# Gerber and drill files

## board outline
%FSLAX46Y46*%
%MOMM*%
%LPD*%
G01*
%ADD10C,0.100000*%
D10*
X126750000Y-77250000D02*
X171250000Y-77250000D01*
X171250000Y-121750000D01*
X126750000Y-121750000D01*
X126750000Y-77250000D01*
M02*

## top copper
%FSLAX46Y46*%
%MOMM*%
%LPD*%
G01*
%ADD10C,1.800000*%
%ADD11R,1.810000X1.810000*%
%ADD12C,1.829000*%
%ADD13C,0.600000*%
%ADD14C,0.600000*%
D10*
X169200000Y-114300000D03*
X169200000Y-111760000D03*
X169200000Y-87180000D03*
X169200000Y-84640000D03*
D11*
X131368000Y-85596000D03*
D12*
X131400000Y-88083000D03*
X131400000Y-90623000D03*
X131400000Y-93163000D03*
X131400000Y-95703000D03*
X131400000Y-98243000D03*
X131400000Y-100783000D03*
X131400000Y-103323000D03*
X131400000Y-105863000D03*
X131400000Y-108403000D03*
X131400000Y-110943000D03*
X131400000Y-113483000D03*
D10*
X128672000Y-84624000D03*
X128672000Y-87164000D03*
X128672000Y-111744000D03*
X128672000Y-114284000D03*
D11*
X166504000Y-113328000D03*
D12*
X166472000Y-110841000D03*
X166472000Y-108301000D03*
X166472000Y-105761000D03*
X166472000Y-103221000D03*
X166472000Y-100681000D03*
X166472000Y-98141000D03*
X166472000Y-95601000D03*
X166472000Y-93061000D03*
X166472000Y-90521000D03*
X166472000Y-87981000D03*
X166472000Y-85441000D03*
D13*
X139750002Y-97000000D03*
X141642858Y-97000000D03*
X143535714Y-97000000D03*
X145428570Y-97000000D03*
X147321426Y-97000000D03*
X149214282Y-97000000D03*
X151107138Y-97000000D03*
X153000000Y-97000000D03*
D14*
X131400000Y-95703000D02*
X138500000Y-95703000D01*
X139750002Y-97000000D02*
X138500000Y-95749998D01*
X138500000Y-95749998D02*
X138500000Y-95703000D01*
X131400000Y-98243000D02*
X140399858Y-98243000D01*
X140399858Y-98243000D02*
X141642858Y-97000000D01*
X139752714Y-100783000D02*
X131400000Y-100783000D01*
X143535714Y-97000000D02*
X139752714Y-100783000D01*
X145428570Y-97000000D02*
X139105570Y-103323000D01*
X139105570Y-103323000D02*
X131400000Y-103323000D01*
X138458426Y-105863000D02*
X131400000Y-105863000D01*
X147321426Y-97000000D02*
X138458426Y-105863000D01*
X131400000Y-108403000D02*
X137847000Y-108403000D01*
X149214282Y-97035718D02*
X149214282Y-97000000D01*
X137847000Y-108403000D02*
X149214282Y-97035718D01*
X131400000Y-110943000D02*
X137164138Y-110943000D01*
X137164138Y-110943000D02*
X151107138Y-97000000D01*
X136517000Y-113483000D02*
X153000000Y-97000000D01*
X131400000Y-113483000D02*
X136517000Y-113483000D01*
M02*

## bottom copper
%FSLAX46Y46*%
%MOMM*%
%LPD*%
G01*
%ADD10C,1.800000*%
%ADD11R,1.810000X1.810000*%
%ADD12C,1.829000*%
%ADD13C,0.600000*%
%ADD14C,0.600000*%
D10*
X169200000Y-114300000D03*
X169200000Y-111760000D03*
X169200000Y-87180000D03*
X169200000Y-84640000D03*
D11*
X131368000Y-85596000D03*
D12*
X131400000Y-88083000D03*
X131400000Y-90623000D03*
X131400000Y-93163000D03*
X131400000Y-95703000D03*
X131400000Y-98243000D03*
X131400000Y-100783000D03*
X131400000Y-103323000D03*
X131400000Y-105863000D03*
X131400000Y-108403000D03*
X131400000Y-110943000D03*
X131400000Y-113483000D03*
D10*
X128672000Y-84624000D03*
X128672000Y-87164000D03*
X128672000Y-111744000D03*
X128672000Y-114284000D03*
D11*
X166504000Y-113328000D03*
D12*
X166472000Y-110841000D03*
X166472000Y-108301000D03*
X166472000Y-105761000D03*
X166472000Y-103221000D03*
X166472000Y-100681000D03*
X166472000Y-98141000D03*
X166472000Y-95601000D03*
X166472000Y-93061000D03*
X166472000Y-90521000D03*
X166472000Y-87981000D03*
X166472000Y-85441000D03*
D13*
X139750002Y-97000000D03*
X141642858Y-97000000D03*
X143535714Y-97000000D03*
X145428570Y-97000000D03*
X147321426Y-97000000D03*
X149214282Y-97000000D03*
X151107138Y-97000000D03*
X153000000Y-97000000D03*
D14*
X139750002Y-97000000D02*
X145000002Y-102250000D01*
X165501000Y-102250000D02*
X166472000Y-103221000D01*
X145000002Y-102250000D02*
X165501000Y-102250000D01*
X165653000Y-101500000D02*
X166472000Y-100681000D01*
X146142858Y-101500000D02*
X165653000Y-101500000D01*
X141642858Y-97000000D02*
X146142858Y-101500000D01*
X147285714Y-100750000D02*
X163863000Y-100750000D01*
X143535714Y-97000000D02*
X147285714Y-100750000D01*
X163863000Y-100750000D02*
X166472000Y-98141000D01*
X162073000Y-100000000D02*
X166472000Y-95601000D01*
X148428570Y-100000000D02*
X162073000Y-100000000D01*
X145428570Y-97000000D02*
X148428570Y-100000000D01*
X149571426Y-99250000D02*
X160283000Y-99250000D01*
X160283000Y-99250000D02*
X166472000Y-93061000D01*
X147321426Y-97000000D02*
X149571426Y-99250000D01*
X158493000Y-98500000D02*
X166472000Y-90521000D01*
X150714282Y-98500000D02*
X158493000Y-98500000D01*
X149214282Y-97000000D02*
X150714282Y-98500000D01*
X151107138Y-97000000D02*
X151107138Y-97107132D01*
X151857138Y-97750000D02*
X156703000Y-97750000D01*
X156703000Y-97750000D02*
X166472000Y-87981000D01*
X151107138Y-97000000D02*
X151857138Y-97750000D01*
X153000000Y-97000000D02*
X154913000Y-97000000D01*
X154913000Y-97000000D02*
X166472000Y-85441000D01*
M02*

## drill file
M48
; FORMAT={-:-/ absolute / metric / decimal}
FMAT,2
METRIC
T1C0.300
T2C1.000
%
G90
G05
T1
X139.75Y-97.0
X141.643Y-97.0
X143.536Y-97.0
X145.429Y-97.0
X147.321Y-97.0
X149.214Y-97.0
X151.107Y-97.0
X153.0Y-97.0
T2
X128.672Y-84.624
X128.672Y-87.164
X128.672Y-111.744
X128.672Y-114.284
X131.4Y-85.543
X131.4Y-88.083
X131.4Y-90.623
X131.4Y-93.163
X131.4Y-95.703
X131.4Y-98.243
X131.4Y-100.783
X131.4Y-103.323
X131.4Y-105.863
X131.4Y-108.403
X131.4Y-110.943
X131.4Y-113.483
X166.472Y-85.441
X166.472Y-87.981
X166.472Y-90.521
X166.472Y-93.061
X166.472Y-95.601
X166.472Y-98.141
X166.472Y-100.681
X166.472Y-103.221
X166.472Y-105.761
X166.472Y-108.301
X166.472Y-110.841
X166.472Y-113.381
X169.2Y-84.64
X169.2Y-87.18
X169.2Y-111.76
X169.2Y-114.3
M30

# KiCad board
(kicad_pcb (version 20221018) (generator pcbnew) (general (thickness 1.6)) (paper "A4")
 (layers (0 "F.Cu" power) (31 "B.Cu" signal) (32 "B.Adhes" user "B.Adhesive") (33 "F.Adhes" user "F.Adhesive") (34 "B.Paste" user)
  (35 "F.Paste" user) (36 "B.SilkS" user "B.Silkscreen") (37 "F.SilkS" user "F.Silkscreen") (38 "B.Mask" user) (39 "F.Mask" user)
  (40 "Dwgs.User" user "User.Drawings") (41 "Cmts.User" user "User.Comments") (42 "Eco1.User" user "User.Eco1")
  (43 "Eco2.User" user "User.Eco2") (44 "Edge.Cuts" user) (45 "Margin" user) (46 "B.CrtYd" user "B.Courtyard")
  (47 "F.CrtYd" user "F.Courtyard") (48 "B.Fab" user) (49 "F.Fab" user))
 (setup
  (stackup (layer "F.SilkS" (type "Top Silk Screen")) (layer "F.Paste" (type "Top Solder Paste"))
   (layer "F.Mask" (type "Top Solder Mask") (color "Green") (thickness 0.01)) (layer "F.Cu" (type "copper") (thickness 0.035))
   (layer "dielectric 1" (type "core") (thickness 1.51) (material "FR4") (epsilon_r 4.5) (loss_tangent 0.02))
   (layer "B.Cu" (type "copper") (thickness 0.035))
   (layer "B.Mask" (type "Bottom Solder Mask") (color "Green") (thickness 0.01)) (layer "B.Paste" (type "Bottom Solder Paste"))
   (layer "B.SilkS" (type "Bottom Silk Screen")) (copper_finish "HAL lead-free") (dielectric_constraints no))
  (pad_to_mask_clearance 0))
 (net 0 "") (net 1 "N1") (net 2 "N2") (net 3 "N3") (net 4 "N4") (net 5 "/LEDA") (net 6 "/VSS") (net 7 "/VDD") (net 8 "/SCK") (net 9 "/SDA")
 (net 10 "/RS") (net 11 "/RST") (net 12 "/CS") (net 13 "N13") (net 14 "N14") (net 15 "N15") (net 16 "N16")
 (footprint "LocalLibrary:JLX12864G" (layer "F.Cu") (at 148.936 99.462 90)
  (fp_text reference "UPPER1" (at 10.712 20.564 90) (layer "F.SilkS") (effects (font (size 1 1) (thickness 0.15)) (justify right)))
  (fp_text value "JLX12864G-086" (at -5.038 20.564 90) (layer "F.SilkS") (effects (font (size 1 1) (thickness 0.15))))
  (pad "" thru_hole circle (at -14.838 20.264 90) (size 1.8 1.8) (drill 1) (layers "*.Cu" "*.Mask"))
  (pad "" thru_hole circle (at -12.298 20.264 90) (size 1.8 1.8) (drill 1) (layers "*.Cu" "*.Mask"))
  (pad "" thru_hole circle (at 12.282 20.264 90) (size 1.8 1.8) (drill 1) (layers "*.Cu" "*.Mask"))
  (pad "" thru_hole circle (at 14.822 20.264 90) (size 1.8 1.8) (drill 1) (layers "*.Cu" "*.Mask"))
  (pad "1" thru_hole rect (at 13.919 -17.536 90) (size 1.81 1.81) (drill 1 (offset -0.053 -0.032)) (layers "*.Cu" "*.Mask") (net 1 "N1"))
  (pad "2" thru_hole circle (at 11.379 -17.536 90) (size 1.829 1.829) (drill 1) (layers "*.Cu" "*.Mask") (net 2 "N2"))
  (pad "3" thru_hole circle (at 8.839 -17.536 90) (size 1.829 1.829) (drill 1) (layers "*.Cu" "*.Mask") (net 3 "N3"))
  (pad "4" thru_hole circle (at 6.299 -17.536 90) (size 1.829 1.829) (drill 1) (layers "*.Cu" "*.Mask") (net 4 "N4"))
  (pad "5" thru_hole circle (at 3.759 -17.536 90) (size 1.829 1.829) (drill 1) (layers "*.Cu" "*.Mask") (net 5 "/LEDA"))
  (pad "6" thru_hole circle (at 1.219 -17.536 90) (size 1.829 1.829) (drill 1) (layers "*.Cu" "*.Mask") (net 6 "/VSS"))
  (pad "7" thru_hole circle (at -1.321 -17.536 90) (size 1.829 1.829) (drill 1) (layers "*.Cu" "*.Mask") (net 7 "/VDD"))
  (pad "8" thru_hole circle (at -3.861 -17.536 90) (size 1.829 1.829) (drill 1) (layers "*.Cu" "*.Mask") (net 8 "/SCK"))
  (pad "9" thru_hole circle (at -6.401 -17.536 90) (size 1.829 1.829) (drill 1) (layers "*.Cu" "*.Mask") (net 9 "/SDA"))
  (pad "10" thru_hole circle (at -8.941 -17.536 90) (size 1.829 1.829) (drill 1) (layers "*.Cu" "*.Mask") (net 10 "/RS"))
  (pad "11" thru_hole circle (at -11.481 -17.536 90) (size 1.829 1.829) (drill 1) (layers "*.Cu" "*.Mask") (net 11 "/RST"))
  (pad "12" thru_hole circle (at -14.021 -17.536 90) (size 1.829 1.829) (drill 1) (layers "*.Cu" "*.Mask") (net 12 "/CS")))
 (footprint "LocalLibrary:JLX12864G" (layer "F.Cu") (at 148.936 99.462 -90)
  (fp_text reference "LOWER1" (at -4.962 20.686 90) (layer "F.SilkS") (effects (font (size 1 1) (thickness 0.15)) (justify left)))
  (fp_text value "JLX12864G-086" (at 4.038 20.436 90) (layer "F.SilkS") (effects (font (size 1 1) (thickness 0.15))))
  (pad "" thru_hole circle (at -14.838 20.264 270) (size 1.8 1.8) (drill 1) (layers "*.Cu" "*.Mask"))
  (pad "" thru_hole circle (at -12.298 20.264 270) (size 1.8 1.8) (drill 1) (layers "*.Cu" "*.Mask"))
  (pad "" thru_hole circle (at 12.282 20.264 270) (size 1.8 1.8) (drill 1) (layers "*.Cu" "*.Mask"))
  (pad "" thru_hole circle (at 14.822 20.264 270) (size 1.8 1.8) (drill 1) (layers "*.Cu" "*.Mask"))
  (pad "1" thru_hole rect (at 13.919 -17.536 270) (size 1.81 1.81) (drill 1 (offset -0.053 -0.032)) (layers "*.Cu" "*.Mask") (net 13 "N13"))
  (pad "2" thru_hole circle (at 11.379 -17.536 270) (size 1.829 1.829) (drill 1) (layers "*.Cu" "*.Mask") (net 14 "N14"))
  (pad "3" thru_hole circle (at 8.839 -17.536 270) (size 1.829 1.829) (drill 1) (layers "*.Cu" "*.Mask") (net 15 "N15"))
  (pad "4" thru_hole circle (at 6.299 -17.536 270) (size 1.829 1.829) (drill 1) (layers "*.Cu" "*.Mask") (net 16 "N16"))
  (pad "5" thru_hole circle (at 3.759 -17.536 270) (size 1.829 1.829) (drill 1) (layers "*.Cu" "*.Mask") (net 5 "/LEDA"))
  (pad "6" thru_hole circle (at 1.219 -17.536 270) (size 1.829 1.829) (drill 1) (layers "*.Cu" "*.Mask") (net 6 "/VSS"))
  (pad "7" thru_hole circle (at -1.321 -17.536 270) (size 1.829 1.829) (drill 1) (layers "*.Cu" "*.Mask") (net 7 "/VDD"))
  (pad "8" thru_hole circle (at -3.861 -17.536 270) (size 1.829 1.829) (drill 1) (layers "*.Cu" "*.Mask") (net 8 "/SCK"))
  (pad "9" thru_hole circle (at -6.401 -17.536 270) (size 1.829 1.829) (drill 1) (layers "*.Cu" "*.Mask") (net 9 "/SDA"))
  (pad "10" thru_hole circle (at -8.941 -17.536 270) (size 1.829 1.829) (drill 1) (layers "*.Cu" "*.Mask") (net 10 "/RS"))
  (pad "11" thru_hole circle (at -11.481 -17.536 270) (size 1.829 1.829) (drill 1) (layers "*.Cu" "*.Mask") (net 11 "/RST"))
  (pad "12" thru_hole circle (at -14.021 -17.536 270) (size 1.829 1.829) (drill 1) (layers "*.Cu" "*.Mask") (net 12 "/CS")))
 (gr_rect (start 126.75 77.25) (end 171.25 121.75) (stroke (width 0.1) (type default)) (fill none) (layer "Edge.Cuts"))
 (segment (start 131.4 95.703) (end 138.5 95.703) (width 0.6) (layer "F.Cu") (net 5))
 (segment (start 139.750002 97) (end 138.5 95.749998) (width 0.6) (layer "F.Cu") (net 5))
 (segment (start 138.5 95.749998) (end 138.5 95.703) (width 0.6) (layer "F.Cu") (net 5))
 (via (at 139.750002 97) (size 0.6) (drill 0.3) (layers "F.Cu" "B.Cu") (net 5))
 (segment (start 139.750002 97) (end 145.000002 102.25) (width 0.6) (layer "B.Cu") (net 5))
 (segment (start 165.501 102.25) (end 166.472 103.221) (width 0.6) (layer "B.Cu") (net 5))
 (segment (start 145.000002 102.25) (end 165.501 102.25) (width 0.6) (layer "B.Cu") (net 5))
 (segment (start 131.4 98.243) (end 140.399858 98.243) (width 0.6) (layer "F.Cu") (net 6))
 (segment (start 140.399858 98.243) (end 141.642858 97) (width 0.6) (layer "F.Cu") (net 6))
 (via (at 141.642858 97) (size 0.6) (drill 0.3) (layers "F.Cu" "B.Cu") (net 6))
 (segment (start 165.653 101.5) (end 166.472 100.681) (width 0.6) (layer "B.Cu") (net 6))
 (segment (start 146.142858 101.5) (end 165.653 101.5) (width 0.6) (layer "B.Cu") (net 6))
 (segment (start 141.642858 97) (end 146.142858 101.5) (width 0.6) (layer "B.Cu") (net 6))
 (segment (start 139.752714 100.783) (end 131.4 100.783) (width 0.6) (layer "F.Cu") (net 7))
 (segment (start 143.535714 97) (end 139.752714 100.783) (width 0.6) (layer "F.Cu") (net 7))
 (via (at 143.535714 97) (size 0.6) (drill 0.3) (layers "F.Cu" "B.Cu") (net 7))
 (segment (start 147.285714 100.75) (end 163.863 100.75) (width 0.6) (layer "B.Cu") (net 7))
 (segment (start 143.535714 97) (end 147.285714 100.75) (width 0.6) (layer "B.Cu") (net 7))
 (segment (start 163.863 100.75) (end 166.472 98.141) (width 0.6) (layer "B.Cu") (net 7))
 (segment (start 145.42857 97) (end 139.10557 103.323) (width 0.6) (layer "F.Cu") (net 8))
 (segment (start 139.10557 103.323) (end 131.4 103.323) (width 0.6) (layer "F.Cu") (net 8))
 (via (at 145.42857 97) (size 0.6) (drill 0.3) (layers "F.Cu" "B.Cu") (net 8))
 (segment (start 162.073 100) (end 166.472 95.601) (width 0.6) (layer "B.Cu") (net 8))
 (segment (start 148.42857 100) (end 162.073 100) (width 0.6) (layer "B.Cu") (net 8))
 (segment (start 145.42857 97) (end 148.42857 100) (width 0.6) (layer "B.Cu") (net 8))
 (segment (start 138.458426 105.863) (end 131.4 105.863) (width 0.6) (layer "F.Cu") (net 9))
 (segment (start 147.321426 97) (end 138.458426 105.863) (width 0.6) (layer "F.Cu") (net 9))
 (via (at 147.321426 97) (size 0.6) (drill 0.3) (layers "F.Cu" "B.Cu") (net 9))
 (segment (start 149.571426 99.25) (end 160.283 99.25) (width 0.6) (layer "B.Cu") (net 9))
 (segment (start 160.283 99.25) (end 166.472 93.061) (width 0.6) (layer "B.Cu") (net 9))
 (segment (start 147.321426 97) (end 149.571426 99.25) (width 0.6) (layer "B.Cu") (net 9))
 (segment (start 131.4 108.403) (end 137.847 108.403) (width 0.6) (layer "F.Cu") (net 10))
 (segment (start 149.214282 97.035718) (end 149.214282 97) (width 0.6) (layer "F.Cu") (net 10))
 (segment (start 137.847 108.403) (end 149.214282 97.035718) (width 0.6) (layer "F.Cu") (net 10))
 (via (at 149.214282 97) (size 0.6) (drill 0.3) (layers "F.Cu" "B.Cu") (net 10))
 (segment (start 158.493 98.5) (end 166.472 90.521) (width 0.6) (layer "B.Cu") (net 10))
 (segment (start 150.714282 98.5) (end 158.493 98.5) (width 0.6) (layer "B.Cu") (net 10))
 (segment (start 149.214282 97) (end 150.714282 98.5) (width 0.6) (layer "B.Cu") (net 10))
 (segment (start 131.4 110.943) (end 137.164138 110.943) (width 0.6) (layer "F.Cu") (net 11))
 (segment (start 137.164138 110.943) (end 151.107138 97) (width 0.6) (layer "F.Cu") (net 11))
 (via (at 151.107138 97) (size 0.6) (drill 0.3) (layers "F.Cu" "B.Cu") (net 11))
 (segment (start 151.107138 97) (end 151.107138 97.107132) (width 0.6) (layer "B.Cu") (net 11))
 (segment (start 151.857138 97.75) (end 156.703 97.75) (width 0.6) (layer "B.Cu") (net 11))
 (segment (start 156.703 97.75) (end 166.472 87.981) (width 0.6) (layer "B.Cu") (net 11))
 (segment (start 151.107138 97) (end 151.857138 97.75) (width 0.6) (layer "B.Cu") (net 11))
 (segment (start 136.517 113.483) (end 153 97) (width 0.6) (layer "F.Cu") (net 12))
 (segment (start 131.4 113.483) (end 136.517 113.483) (width 0.6) (layer "F.Cu") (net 12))
 (via (at 153 97) (size 0.6) (drill 0.3) (layers "F.Cu" "B.Cu") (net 12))
 (segment (start 153 97) (end 154.913 97) (width 0.6) (layer "B.Cu") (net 12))
 (segment (start 154.913 97) (end 166.472 85.441) (width 0.6) (layer "B.Cu") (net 12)))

